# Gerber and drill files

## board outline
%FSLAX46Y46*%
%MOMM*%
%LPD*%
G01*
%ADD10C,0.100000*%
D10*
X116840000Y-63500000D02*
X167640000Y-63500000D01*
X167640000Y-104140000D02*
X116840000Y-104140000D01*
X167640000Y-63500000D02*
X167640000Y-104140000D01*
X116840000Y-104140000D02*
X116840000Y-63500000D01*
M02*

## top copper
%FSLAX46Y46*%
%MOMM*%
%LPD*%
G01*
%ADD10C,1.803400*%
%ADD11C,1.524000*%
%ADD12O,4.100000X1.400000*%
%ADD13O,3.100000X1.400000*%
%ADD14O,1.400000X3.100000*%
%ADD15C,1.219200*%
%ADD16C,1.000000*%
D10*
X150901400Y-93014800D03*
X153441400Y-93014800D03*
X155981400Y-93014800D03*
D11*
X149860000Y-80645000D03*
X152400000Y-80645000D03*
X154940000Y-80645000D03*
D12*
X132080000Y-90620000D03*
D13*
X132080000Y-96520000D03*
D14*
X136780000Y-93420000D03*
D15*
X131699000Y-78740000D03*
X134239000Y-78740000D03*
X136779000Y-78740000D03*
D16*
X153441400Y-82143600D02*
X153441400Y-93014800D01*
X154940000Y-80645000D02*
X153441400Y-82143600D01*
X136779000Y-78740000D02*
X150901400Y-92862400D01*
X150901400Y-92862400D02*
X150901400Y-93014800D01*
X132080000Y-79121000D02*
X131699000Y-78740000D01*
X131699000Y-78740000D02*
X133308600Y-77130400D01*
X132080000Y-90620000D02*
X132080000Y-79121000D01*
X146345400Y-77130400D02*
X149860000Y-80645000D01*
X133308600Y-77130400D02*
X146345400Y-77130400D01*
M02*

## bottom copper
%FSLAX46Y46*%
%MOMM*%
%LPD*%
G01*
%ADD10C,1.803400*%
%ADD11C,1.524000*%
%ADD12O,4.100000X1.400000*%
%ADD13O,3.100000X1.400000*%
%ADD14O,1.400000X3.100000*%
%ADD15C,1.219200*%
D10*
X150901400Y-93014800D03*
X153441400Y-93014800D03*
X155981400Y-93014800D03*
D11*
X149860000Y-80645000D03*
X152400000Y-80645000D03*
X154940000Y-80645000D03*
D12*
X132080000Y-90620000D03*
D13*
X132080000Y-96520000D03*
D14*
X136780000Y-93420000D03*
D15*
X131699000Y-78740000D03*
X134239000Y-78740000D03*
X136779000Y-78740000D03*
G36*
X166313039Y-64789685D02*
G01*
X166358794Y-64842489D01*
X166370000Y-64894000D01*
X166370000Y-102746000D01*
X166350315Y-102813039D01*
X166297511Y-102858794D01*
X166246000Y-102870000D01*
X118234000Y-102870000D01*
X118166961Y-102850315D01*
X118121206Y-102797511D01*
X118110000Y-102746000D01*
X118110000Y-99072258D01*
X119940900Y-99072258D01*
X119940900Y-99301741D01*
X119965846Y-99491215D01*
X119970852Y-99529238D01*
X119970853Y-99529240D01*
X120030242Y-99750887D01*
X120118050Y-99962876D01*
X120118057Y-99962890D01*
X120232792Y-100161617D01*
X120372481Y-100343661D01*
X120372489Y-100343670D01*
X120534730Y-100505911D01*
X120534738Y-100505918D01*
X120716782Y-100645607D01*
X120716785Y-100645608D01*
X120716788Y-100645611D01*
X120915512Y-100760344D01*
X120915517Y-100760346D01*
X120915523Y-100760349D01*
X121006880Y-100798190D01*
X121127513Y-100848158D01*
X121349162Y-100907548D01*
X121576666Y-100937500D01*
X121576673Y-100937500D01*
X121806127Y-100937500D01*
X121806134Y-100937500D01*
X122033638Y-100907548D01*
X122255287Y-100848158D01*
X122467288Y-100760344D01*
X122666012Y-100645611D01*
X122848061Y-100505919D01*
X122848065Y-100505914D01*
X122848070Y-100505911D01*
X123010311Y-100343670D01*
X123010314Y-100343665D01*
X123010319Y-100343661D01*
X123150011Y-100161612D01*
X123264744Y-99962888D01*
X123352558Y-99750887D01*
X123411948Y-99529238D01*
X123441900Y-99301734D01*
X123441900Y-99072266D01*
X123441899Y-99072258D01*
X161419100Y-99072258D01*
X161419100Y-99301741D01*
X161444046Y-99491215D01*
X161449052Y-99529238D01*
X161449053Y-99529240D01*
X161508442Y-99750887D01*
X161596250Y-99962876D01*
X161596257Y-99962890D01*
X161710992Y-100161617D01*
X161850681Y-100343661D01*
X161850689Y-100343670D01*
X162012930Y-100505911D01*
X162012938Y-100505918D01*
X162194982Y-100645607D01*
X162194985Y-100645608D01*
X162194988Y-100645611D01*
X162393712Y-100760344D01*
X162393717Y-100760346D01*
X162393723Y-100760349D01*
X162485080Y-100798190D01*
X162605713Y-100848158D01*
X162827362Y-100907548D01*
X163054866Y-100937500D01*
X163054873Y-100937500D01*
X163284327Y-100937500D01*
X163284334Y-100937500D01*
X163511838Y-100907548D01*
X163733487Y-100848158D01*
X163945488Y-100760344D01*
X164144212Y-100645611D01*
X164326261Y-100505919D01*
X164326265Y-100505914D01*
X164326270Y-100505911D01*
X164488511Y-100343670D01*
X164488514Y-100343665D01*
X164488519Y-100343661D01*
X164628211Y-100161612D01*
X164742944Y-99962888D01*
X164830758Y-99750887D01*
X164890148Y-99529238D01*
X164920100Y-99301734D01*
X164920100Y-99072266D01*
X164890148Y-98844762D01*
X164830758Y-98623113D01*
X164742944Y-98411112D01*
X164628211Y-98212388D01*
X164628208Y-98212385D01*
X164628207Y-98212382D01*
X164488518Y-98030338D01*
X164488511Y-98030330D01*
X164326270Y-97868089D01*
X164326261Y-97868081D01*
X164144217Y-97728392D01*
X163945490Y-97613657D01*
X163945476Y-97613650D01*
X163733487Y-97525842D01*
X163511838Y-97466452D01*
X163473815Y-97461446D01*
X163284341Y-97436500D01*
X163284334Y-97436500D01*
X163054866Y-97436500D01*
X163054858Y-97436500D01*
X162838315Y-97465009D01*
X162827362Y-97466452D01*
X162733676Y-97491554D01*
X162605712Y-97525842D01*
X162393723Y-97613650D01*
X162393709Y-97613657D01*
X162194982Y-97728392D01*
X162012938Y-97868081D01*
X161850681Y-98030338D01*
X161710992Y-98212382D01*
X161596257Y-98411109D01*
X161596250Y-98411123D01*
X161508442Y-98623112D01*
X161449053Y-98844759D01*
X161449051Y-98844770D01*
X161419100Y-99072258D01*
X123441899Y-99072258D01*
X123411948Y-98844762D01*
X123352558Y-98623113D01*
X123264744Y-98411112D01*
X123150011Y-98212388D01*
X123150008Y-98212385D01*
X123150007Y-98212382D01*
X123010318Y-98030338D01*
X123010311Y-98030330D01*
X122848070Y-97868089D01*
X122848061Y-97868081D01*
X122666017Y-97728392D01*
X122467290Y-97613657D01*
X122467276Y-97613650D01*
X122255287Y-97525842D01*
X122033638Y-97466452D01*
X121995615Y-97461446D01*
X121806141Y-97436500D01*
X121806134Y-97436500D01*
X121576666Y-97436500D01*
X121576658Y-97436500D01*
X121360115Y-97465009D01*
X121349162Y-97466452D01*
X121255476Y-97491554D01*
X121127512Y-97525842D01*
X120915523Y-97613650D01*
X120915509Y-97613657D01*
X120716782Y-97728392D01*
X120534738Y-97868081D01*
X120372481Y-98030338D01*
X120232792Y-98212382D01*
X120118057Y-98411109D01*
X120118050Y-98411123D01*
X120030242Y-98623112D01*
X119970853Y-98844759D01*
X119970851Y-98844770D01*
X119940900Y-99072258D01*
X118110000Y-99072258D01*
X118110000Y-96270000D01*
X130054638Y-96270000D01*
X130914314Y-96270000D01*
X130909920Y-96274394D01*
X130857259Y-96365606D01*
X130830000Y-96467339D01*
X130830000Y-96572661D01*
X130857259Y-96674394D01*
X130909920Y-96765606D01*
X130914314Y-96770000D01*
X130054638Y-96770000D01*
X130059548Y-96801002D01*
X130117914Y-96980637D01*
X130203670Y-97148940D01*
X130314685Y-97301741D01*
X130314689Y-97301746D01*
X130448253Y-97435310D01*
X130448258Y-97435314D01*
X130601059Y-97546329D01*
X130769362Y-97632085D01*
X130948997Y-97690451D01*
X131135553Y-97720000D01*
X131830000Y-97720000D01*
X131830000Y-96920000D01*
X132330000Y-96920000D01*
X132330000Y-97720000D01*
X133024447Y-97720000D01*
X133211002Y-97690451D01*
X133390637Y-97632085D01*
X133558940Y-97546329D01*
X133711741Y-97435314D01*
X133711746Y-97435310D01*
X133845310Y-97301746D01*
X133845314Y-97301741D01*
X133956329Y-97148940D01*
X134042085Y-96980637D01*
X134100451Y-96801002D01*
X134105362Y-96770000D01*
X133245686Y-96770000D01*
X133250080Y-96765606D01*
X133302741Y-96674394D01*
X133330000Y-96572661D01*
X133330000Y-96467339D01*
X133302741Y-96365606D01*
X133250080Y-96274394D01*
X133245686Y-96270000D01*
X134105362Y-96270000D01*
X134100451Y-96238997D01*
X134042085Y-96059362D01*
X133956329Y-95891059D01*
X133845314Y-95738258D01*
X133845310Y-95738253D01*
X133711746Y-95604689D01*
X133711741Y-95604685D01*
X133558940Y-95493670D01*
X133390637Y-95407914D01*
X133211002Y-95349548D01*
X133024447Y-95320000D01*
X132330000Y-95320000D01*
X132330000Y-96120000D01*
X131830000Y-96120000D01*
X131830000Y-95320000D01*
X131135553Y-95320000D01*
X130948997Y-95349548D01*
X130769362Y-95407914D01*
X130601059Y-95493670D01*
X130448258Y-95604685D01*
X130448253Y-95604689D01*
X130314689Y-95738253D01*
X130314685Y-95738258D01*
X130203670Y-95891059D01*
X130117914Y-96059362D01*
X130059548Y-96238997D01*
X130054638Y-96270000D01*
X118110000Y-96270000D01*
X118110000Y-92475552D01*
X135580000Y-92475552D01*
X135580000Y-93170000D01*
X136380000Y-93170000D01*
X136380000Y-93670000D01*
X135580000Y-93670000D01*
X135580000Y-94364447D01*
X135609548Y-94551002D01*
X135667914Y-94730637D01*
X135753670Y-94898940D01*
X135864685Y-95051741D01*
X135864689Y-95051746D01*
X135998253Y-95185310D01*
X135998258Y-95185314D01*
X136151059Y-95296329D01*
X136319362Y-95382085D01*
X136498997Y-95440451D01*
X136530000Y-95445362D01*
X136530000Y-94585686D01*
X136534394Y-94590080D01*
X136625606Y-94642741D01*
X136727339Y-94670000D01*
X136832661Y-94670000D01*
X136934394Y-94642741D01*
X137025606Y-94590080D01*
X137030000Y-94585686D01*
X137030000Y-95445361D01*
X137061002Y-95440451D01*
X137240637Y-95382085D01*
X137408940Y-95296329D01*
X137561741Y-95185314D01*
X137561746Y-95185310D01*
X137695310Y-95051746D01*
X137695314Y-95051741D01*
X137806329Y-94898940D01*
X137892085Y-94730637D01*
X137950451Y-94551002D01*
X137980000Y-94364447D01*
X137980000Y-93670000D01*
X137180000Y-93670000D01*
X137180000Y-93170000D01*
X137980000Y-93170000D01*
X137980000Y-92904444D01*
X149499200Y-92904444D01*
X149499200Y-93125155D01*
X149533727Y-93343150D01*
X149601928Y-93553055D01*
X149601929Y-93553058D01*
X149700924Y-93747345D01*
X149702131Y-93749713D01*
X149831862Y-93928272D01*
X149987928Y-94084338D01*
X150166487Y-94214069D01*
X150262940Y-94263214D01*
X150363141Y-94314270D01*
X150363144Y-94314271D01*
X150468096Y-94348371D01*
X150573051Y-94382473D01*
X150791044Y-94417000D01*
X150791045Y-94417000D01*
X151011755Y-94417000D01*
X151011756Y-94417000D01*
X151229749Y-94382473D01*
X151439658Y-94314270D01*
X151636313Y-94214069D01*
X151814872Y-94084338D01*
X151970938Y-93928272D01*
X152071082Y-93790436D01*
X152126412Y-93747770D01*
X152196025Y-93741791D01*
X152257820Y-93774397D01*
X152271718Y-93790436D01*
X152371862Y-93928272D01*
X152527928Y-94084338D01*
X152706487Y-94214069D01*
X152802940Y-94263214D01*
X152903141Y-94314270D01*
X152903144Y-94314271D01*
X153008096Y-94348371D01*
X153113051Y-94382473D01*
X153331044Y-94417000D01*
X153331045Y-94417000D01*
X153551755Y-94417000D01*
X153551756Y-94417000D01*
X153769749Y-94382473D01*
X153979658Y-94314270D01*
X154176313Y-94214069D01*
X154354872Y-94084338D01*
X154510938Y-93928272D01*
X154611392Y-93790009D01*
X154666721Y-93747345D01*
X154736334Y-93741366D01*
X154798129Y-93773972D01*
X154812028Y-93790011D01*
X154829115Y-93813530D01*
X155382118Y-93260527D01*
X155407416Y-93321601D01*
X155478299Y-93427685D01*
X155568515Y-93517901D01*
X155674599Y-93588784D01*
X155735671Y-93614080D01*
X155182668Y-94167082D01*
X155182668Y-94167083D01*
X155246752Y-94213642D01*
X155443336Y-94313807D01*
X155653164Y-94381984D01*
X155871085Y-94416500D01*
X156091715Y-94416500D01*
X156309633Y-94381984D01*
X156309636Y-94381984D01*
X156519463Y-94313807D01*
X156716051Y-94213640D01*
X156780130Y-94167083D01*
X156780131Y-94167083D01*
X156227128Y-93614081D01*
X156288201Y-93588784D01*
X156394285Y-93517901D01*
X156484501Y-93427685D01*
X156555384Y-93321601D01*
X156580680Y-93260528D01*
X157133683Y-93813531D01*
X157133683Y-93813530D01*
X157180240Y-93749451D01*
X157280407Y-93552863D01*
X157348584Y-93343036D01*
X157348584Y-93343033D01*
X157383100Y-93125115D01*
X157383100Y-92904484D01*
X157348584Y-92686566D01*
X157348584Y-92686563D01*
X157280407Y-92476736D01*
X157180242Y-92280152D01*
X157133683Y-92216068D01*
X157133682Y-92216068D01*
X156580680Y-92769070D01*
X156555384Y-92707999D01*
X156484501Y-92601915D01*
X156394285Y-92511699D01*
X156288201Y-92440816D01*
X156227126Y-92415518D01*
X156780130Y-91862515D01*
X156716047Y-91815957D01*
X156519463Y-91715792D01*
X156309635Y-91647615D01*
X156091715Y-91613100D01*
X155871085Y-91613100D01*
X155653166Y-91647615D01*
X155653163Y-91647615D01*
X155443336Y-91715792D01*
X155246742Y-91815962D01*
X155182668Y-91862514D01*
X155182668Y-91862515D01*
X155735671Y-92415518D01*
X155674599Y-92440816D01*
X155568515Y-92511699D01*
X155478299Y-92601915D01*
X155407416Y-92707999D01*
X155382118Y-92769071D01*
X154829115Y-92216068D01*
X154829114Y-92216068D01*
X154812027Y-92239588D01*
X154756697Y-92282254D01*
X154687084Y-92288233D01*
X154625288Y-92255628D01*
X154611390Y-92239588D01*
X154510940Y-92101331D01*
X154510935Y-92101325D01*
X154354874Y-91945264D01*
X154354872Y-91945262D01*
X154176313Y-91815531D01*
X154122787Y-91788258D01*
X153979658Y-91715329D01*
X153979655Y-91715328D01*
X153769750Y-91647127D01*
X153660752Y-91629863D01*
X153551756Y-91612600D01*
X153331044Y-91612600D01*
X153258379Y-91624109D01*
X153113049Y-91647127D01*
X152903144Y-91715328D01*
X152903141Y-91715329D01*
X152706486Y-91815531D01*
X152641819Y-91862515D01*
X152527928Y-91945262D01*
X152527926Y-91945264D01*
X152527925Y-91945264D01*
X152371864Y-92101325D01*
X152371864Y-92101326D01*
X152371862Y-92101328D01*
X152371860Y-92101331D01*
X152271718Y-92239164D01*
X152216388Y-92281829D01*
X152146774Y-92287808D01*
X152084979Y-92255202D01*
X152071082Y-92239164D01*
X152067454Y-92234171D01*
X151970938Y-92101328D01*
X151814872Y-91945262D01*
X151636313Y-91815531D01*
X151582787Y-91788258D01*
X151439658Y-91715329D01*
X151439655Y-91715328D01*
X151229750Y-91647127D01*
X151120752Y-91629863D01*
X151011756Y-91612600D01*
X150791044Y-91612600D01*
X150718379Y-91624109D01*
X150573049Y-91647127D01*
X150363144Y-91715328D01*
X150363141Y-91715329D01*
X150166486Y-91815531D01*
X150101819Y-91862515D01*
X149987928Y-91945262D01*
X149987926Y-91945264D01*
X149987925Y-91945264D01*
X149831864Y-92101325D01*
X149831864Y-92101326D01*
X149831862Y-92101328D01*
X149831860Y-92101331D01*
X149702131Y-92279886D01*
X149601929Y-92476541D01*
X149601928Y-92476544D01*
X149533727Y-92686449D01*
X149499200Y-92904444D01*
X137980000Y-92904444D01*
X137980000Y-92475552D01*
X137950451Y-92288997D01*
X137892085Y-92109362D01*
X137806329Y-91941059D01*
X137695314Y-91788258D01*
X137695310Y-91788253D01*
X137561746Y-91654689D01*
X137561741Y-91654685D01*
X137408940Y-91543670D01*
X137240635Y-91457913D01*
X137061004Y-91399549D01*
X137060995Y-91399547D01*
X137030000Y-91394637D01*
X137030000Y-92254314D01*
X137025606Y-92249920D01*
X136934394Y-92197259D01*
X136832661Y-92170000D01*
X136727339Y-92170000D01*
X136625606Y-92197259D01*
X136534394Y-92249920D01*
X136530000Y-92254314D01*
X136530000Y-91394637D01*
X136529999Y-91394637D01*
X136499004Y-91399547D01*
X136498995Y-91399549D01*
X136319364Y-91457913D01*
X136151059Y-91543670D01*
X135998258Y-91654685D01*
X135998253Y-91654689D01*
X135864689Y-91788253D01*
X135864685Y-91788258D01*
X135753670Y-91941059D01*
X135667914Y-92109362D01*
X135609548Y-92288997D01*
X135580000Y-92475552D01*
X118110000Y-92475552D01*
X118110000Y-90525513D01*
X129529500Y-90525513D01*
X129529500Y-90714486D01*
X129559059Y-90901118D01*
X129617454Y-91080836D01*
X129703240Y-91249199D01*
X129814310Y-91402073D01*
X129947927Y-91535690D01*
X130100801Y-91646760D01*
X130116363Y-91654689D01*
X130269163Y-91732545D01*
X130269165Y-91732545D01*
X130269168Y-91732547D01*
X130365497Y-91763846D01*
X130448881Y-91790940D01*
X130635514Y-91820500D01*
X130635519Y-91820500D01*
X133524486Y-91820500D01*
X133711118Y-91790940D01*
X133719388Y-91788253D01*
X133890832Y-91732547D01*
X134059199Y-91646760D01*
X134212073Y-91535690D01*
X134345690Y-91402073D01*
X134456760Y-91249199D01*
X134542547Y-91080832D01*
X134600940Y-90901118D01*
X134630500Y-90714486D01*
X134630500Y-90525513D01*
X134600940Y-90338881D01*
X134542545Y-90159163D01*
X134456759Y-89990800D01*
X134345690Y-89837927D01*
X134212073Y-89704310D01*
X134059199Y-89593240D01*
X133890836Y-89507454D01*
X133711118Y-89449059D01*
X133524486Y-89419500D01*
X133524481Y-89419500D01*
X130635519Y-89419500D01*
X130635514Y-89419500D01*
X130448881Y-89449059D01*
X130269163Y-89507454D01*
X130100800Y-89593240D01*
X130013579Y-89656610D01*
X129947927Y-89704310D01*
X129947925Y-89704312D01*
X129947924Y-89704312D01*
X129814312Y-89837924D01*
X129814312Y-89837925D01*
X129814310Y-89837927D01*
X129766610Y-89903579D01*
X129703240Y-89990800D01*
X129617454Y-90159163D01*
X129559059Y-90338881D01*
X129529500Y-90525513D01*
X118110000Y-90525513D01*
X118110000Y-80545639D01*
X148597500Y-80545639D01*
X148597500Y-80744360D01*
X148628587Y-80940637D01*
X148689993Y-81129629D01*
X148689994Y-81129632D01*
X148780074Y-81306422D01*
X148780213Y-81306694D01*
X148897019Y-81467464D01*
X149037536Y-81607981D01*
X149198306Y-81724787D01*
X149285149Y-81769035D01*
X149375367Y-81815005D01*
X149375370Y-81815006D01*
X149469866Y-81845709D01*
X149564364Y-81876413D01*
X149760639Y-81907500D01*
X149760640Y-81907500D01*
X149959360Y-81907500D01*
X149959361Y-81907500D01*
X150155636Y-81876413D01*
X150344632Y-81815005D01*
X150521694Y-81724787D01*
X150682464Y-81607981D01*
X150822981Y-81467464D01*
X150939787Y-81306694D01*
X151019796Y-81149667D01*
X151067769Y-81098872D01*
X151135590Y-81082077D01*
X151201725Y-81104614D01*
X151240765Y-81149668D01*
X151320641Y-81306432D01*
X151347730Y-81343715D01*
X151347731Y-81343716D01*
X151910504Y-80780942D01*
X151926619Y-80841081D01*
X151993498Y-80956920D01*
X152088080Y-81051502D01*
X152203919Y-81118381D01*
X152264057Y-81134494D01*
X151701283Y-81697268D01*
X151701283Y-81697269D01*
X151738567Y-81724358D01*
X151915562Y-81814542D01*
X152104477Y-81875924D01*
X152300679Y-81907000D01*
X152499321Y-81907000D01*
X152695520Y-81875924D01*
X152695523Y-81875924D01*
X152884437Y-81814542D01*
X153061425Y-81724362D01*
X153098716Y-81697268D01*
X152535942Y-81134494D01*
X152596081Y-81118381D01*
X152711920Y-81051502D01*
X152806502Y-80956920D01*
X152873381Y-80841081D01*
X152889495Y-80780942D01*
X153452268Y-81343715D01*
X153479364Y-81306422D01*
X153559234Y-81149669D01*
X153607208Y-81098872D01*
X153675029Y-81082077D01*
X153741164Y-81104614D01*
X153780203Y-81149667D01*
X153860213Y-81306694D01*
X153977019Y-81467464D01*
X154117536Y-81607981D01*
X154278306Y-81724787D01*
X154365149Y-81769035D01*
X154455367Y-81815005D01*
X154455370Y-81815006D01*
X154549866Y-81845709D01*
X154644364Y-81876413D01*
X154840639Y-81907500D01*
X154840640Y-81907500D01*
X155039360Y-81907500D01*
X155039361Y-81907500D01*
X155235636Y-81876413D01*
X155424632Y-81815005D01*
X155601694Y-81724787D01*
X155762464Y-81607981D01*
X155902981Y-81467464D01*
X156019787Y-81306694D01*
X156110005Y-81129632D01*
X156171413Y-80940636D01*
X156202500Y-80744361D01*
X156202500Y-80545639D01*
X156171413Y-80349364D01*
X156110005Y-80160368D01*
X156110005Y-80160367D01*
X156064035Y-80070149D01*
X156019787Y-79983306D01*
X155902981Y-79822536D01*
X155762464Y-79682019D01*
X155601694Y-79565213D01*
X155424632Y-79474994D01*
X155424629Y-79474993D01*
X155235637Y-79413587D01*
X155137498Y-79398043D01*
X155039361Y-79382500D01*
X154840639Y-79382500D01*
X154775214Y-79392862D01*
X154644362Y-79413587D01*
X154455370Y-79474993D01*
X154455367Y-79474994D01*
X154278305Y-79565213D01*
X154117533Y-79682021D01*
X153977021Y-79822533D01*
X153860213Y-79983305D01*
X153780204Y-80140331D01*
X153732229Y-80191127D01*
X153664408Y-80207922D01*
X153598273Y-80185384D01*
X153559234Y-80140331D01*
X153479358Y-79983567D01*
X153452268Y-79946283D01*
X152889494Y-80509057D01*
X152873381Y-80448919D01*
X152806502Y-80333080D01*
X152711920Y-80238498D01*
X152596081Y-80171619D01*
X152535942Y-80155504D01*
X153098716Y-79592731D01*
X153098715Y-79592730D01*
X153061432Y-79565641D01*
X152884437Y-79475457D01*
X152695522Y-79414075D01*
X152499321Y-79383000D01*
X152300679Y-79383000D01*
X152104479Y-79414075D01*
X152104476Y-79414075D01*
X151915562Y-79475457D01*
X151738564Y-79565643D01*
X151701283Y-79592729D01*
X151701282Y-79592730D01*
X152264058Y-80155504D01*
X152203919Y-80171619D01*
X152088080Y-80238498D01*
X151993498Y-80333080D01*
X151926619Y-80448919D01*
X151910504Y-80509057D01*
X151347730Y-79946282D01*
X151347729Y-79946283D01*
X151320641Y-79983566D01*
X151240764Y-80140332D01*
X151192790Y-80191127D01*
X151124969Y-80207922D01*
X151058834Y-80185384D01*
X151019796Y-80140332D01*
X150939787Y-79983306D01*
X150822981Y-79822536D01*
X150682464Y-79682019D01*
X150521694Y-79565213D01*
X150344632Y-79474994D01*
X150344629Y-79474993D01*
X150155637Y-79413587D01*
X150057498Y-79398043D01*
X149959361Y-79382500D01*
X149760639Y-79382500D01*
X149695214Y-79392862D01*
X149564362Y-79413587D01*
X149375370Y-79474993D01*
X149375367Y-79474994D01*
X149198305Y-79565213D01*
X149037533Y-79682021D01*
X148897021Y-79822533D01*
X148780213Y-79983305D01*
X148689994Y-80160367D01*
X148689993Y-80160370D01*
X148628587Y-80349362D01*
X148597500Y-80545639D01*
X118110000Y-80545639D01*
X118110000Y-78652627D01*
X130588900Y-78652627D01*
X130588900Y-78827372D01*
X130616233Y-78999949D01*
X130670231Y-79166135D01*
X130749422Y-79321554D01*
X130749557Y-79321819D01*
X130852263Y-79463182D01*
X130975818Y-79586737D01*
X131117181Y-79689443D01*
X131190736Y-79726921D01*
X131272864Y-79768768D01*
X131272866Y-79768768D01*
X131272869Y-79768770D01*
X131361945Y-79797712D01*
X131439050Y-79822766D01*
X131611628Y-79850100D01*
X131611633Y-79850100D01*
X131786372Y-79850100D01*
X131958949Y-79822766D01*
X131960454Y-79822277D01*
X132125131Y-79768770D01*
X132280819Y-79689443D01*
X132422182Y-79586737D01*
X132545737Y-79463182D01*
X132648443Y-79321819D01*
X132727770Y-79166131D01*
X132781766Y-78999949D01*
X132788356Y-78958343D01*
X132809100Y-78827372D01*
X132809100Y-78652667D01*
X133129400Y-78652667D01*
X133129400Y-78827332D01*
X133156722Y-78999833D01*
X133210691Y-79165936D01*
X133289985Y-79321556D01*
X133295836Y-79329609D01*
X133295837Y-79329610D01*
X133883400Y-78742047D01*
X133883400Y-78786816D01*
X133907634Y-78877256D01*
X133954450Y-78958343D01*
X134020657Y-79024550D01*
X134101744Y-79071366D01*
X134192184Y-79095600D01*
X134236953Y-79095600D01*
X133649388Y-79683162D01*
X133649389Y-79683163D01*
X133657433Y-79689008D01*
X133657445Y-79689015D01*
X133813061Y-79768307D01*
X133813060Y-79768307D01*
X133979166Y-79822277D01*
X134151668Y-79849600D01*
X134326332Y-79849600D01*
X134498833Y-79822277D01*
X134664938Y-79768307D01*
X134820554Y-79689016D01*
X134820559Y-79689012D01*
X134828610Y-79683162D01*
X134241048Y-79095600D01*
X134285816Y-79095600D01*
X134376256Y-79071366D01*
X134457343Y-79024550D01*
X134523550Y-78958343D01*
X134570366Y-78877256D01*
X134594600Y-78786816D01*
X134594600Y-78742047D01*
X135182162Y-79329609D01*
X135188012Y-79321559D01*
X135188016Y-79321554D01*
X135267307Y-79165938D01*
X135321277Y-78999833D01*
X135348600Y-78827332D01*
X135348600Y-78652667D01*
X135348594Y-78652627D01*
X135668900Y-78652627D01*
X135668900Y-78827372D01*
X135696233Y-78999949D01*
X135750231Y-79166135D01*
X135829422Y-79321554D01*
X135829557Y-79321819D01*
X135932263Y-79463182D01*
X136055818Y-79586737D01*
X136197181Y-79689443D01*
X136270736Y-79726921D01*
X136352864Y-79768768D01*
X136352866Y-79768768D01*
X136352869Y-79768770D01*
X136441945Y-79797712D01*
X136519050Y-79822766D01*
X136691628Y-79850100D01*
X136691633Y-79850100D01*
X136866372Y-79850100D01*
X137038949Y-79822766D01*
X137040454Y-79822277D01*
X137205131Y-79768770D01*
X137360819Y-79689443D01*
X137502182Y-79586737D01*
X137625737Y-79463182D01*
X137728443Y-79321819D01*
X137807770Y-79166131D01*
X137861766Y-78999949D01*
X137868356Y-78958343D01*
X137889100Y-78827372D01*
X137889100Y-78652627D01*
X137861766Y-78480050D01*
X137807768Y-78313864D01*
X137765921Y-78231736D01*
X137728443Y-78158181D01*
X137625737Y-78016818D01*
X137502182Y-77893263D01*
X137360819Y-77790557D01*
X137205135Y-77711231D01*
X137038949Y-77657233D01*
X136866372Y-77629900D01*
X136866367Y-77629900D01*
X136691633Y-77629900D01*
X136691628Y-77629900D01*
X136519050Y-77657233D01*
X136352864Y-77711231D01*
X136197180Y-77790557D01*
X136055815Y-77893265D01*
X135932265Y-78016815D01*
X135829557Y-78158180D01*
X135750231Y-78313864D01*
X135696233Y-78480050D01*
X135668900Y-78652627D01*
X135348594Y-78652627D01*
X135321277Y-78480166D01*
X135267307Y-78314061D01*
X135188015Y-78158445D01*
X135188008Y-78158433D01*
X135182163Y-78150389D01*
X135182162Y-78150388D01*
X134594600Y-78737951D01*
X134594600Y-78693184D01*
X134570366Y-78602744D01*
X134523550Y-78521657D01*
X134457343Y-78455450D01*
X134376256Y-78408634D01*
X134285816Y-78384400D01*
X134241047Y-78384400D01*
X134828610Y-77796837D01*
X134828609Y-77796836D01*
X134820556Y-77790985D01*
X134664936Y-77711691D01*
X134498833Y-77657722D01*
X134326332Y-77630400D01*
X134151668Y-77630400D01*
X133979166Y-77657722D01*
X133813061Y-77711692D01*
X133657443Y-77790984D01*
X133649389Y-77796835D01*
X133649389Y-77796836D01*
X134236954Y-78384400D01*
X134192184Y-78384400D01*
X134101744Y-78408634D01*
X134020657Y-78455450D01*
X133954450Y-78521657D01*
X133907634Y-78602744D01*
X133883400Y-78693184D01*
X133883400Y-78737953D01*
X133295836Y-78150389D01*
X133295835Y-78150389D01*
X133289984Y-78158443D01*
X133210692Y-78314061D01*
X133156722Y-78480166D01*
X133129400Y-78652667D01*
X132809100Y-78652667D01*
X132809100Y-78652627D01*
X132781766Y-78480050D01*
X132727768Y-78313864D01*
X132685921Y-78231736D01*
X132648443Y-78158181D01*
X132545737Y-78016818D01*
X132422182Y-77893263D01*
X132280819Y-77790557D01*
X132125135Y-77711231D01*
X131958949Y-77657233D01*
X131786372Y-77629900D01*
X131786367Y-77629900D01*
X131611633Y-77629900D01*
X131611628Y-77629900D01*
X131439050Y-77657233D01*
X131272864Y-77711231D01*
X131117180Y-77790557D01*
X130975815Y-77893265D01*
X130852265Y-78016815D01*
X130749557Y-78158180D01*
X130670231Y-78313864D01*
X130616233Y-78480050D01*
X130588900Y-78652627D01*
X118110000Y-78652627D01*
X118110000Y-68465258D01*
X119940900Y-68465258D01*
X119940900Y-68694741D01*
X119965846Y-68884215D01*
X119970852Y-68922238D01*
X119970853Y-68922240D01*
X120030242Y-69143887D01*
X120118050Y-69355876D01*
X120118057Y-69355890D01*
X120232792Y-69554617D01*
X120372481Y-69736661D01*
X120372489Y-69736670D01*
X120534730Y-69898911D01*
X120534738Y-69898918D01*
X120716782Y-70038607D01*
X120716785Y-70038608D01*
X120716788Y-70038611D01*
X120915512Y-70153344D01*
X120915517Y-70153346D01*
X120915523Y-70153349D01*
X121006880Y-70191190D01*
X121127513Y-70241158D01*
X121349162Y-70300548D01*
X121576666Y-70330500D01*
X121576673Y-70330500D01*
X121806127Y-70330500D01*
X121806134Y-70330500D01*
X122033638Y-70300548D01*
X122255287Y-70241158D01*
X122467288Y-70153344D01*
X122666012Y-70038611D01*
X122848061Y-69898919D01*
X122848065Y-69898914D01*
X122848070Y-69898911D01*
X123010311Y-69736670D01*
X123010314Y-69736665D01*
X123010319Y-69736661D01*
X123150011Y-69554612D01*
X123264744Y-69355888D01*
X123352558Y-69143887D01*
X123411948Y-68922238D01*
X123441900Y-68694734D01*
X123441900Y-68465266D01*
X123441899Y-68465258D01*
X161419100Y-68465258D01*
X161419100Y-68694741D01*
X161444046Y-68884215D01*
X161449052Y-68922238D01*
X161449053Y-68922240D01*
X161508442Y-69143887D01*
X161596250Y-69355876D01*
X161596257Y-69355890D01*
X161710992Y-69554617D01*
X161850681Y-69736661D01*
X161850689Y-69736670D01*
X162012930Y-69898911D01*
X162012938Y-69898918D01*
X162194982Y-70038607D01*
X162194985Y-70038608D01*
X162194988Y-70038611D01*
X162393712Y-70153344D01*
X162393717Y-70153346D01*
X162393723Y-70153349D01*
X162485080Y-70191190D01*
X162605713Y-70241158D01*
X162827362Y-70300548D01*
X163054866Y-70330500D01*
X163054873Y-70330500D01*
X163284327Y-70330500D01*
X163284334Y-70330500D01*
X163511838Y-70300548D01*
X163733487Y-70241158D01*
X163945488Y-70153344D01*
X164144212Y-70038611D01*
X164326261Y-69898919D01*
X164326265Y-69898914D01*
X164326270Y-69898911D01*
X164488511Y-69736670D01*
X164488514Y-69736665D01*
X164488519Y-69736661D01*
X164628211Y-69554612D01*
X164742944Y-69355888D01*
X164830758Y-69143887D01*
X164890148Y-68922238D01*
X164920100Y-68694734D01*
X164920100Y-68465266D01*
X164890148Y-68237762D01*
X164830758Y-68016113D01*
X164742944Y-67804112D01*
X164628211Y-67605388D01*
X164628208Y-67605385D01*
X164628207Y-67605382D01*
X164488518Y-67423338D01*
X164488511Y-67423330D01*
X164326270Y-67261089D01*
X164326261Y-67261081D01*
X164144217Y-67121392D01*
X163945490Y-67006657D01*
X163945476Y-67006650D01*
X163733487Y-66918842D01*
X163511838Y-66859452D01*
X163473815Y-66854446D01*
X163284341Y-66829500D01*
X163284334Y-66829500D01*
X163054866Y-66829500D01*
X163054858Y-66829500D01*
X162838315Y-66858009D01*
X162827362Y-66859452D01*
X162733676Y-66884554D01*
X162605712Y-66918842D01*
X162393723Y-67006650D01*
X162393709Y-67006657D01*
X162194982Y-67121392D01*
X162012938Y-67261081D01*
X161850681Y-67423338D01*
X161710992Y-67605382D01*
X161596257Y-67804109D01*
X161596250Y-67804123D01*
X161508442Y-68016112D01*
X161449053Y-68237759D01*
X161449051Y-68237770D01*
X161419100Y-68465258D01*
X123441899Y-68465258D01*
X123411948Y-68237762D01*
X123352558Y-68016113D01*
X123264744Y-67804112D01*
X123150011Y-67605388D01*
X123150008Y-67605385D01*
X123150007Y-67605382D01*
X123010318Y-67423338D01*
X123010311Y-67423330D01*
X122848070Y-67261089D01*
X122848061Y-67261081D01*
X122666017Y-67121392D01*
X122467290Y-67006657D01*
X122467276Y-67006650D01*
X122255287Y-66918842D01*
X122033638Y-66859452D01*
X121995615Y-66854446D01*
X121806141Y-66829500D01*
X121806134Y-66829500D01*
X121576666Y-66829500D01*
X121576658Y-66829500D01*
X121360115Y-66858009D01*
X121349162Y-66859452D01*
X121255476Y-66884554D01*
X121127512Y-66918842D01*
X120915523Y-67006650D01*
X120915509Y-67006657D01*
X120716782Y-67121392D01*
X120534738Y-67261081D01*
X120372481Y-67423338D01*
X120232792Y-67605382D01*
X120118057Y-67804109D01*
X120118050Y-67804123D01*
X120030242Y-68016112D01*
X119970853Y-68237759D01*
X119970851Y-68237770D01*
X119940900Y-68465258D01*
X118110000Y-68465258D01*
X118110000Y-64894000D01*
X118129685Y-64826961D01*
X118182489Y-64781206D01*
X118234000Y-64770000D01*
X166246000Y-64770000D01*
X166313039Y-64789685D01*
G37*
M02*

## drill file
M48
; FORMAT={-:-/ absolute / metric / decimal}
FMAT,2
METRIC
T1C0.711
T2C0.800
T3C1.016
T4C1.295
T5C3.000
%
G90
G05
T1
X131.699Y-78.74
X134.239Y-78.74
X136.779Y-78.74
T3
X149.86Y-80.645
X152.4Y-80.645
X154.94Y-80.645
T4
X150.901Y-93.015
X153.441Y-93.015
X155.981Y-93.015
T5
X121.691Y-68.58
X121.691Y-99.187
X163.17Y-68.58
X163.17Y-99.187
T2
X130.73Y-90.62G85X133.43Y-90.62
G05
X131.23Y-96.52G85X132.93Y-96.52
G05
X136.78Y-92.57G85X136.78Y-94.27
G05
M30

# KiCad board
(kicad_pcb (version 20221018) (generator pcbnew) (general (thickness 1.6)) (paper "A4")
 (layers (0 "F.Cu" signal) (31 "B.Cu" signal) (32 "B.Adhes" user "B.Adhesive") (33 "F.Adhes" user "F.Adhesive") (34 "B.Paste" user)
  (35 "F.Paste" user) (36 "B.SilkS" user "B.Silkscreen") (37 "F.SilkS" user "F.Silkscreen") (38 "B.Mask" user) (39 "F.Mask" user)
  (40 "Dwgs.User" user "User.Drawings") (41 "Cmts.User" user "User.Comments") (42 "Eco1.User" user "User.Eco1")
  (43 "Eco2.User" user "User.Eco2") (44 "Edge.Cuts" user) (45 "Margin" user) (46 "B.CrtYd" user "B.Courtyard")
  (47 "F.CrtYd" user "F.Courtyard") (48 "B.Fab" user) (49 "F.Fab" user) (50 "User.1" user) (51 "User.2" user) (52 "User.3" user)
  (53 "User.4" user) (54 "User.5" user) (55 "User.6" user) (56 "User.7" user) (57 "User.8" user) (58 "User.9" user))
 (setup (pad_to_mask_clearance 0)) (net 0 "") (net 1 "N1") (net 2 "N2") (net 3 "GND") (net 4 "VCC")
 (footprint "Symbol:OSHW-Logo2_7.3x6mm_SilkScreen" (layer "F.Cu") (at 123.19 83.82)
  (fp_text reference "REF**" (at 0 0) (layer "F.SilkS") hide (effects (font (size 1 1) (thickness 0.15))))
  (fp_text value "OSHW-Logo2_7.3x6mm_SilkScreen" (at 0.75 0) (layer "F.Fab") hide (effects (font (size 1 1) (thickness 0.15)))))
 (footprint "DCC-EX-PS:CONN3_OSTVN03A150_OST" (layer "F.Cu") (at 150.9014 93.0148)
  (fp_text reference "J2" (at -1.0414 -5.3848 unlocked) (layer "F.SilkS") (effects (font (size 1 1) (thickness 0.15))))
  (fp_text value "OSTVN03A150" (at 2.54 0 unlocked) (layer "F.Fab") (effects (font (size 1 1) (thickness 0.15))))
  (pad "1" thru_hole circle (at 0 0) (size 1.8034 1.8034) (drill 1.2954) (layers "*.Cu" "*.Mask") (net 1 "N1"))
  (pad "2" thru_hole circle (at 2.54 0) (size 1.8034 1.8034) (drill 1.2954) (layers "*.Cu" "*.Mask") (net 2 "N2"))
  (pad "3" thru_hole circle (at 5.08 0) (size 1.8034 1.8034) (drill 1.2954) (layers "*.Cu" "*.Mask") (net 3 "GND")))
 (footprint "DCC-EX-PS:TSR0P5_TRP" (layer "F.Cu") (at 149.86 80.645)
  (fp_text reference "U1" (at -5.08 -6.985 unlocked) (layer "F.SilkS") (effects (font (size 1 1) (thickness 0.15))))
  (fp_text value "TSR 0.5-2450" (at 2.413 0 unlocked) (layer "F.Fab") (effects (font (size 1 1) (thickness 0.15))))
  (pad "1" thru_hole circle (at 0 0) (size 1.524 1.524) (drill 1.016) (layers "*.Cu" "*.Mask") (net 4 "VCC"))
  (pad "2" thru_hole circle (at 2.54 0) (size 1.524 1.524) (drill 1.016) (layers "*.Cu" "*.Mask") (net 3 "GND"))
  (pad "3" thru_hole circle (at 5.08 0) (size 1.524 1.524) (drill 1.016) (layers "*.Cu" "*.Mask") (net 2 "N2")))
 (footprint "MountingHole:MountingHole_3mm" (layer "F.Cu") (at 163.1696 99.187)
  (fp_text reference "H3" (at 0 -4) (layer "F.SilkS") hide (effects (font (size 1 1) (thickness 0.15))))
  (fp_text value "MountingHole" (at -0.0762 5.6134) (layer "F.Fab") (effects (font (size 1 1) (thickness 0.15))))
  (pad "" np_thru_hole circle (at 0 0) (size 3 3) (drill 3) (layers "*.Cu" "*.Mask")))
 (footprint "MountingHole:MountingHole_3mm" (layer "F.Cu") (at 121.6914 68.58)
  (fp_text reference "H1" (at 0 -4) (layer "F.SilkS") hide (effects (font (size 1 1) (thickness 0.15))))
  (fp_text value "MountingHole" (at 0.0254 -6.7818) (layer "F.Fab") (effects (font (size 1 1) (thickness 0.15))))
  (pad "" np_thru_hole circle (at 0 0) (size 3 3) (drill 3) (layers "*.Cu" "*.Mask")))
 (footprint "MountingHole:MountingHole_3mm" (layer "F.Cu") (at 163.1696 68.58)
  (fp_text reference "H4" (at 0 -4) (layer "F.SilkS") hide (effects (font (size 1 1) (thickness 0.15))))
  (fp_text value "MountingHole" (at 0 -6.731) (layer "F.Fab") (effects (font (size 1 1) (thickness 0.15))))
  (pad "" np_thru_hole circle (at 0 0) (size 3 3) (drill 3) (layers "*.Cu" "*.Mask")))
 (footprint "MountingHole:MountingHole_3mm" (layer "F.Cu") (at 121.6914 99.187)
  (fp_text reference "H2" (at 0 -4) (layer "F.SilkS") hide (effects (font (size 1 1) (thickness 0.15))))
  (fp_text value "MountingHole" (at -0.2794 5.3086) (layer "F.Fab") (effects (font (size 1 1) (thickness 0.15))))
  (pad "" np_thru_hole circle (at 0 0) (size 3 3) (drill 3) (layers "*.Cu" "*.Mask")))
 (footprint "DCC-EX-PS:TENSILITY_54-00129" (layer "F.Cu") (at 132.08 96.52)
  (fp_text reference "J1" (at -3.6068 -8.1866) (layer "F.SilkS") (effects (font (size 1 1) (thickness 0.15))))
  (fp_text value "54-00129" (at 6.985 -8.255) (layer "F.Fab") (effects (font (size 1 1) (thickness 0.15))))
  (pad "A" thru_hole oval (at 0 -5.9) (size 4.1 1.4) (drill oval 3.5 0.8) (layers "*.Cu" "*.Mask") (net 4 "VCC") (solder_mask_margin 0.102))
  (pad "B" thru_hole oval (at 0 0) (size 3.1 1.4) (drill oval 2.5 0.8) (layers "*.Cu" "*.Mask") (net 3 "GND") (solder_mask_margin 0.102))
  (pad "C" thru_hole oval (at 4.7 -3.1) (size 1.4 3.1) (drill oval 0.8 2.5) (layers "*.Cu" "*.Mask") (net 3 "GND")
   (solder_mask_margin 0.102)))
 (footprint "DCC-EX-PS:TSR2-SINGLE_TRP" (layer "F.Cu") (at 131.699 78.74)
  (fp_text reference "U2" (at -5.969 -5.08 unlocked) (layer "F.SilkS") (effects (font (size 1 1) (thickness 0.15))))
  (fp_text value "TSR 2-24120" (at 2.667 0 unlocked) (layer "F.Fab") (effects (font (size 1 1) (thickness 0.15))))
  (pad "1" thru_hole circle (at 0 0) (size 1.2192 1.2192) (drill 0.7112) (layers "*.Cu" "*.Mask") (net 4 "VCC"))
  (pad "2" thru_hole circle (at 2.54 0) (size 1.2192 1.2192) (drill 0.7112) (layers "*.Cu" "*.Mask") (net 3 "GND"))
  (pad "3" thru_hole circle (at 5.08 0) (size 1.2192 1.2192) (drill 0.7112) (layers "*.Cu" "*.Mask") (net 1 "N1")))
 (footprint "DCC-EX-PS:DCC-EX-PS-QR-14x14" (layer "B.Cu") (at 149.86 72.39 180)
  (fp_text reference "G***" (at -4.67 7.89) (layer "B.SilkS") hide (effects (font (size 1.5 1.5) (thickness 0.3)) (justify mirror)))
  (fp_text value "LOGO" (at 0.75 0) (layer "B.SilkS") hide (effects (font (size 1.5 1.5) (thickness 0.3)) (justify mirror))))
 (gr_line (start 116.84 63.5) (end 167.64 63.5) (stroke (width 0.1) (type default)) (layer "Edge.Cuts"))
 (gr_line (start 167.64 104.14) (end 116.84 104.14) (stroke (width 0.1) (type default)) (layer "Edge.Cuts"))
 (gr_line (start 167.64 63.5) (end 167.64 104.14) (stroke (width 0.1) (type default)) (layer "Edge.Cuts"))
 (gr_line (start 116.84 104.14) (end 116.84 63.5) (stroke (width 0.1) (type default)) (layer "Edge.Cuts"))
 (segment (start 153.4414 82.1436) (end 153.4414 93.0148) (width 1) (layer "F.Cu") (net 2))
 (segment (start 154.94 80.645) (end 153.4414 82.1436) (width 1) (layer "F.Cu") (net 2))
 (segment (start 136.779 78.74) (end 150.9014 92.8624) (width 1) (layer "F.Cu") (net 1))
 (segment (start 150.9014 92.8624) (end 150.9014 93.0148) (width 1) (layer "F.Cu") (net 1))
 (segment (start 132.08 79.121) (end 131.699 78.74) (width 1) (layer "F.Cu") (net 4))
 (segment (start 131.699 78.74) (end 133.3086 77.1304) (width 1) (layer "F.Cu") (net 4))
 (segment (start 132.08 90.62) (end 132.08 79.121) (width 1) (layer "F.Cu") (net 4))
 (segment (start 146.3454 77.1304) (end 149.86 80.645) (width 1) (layer "F.Cu") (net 4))
 (segment (start 133.3086 77.1304) (end 146.3454 77.1304) (width 1) (layer "F.Cu") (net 4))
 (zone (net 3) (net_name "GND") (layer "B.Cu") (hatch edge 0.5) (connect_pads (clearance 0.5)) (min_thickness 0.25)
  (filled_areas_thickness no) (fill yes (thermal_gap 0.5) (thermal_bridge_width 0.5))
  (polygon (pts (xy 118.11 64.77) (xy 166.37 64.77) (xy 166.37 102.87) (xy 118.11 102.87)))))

